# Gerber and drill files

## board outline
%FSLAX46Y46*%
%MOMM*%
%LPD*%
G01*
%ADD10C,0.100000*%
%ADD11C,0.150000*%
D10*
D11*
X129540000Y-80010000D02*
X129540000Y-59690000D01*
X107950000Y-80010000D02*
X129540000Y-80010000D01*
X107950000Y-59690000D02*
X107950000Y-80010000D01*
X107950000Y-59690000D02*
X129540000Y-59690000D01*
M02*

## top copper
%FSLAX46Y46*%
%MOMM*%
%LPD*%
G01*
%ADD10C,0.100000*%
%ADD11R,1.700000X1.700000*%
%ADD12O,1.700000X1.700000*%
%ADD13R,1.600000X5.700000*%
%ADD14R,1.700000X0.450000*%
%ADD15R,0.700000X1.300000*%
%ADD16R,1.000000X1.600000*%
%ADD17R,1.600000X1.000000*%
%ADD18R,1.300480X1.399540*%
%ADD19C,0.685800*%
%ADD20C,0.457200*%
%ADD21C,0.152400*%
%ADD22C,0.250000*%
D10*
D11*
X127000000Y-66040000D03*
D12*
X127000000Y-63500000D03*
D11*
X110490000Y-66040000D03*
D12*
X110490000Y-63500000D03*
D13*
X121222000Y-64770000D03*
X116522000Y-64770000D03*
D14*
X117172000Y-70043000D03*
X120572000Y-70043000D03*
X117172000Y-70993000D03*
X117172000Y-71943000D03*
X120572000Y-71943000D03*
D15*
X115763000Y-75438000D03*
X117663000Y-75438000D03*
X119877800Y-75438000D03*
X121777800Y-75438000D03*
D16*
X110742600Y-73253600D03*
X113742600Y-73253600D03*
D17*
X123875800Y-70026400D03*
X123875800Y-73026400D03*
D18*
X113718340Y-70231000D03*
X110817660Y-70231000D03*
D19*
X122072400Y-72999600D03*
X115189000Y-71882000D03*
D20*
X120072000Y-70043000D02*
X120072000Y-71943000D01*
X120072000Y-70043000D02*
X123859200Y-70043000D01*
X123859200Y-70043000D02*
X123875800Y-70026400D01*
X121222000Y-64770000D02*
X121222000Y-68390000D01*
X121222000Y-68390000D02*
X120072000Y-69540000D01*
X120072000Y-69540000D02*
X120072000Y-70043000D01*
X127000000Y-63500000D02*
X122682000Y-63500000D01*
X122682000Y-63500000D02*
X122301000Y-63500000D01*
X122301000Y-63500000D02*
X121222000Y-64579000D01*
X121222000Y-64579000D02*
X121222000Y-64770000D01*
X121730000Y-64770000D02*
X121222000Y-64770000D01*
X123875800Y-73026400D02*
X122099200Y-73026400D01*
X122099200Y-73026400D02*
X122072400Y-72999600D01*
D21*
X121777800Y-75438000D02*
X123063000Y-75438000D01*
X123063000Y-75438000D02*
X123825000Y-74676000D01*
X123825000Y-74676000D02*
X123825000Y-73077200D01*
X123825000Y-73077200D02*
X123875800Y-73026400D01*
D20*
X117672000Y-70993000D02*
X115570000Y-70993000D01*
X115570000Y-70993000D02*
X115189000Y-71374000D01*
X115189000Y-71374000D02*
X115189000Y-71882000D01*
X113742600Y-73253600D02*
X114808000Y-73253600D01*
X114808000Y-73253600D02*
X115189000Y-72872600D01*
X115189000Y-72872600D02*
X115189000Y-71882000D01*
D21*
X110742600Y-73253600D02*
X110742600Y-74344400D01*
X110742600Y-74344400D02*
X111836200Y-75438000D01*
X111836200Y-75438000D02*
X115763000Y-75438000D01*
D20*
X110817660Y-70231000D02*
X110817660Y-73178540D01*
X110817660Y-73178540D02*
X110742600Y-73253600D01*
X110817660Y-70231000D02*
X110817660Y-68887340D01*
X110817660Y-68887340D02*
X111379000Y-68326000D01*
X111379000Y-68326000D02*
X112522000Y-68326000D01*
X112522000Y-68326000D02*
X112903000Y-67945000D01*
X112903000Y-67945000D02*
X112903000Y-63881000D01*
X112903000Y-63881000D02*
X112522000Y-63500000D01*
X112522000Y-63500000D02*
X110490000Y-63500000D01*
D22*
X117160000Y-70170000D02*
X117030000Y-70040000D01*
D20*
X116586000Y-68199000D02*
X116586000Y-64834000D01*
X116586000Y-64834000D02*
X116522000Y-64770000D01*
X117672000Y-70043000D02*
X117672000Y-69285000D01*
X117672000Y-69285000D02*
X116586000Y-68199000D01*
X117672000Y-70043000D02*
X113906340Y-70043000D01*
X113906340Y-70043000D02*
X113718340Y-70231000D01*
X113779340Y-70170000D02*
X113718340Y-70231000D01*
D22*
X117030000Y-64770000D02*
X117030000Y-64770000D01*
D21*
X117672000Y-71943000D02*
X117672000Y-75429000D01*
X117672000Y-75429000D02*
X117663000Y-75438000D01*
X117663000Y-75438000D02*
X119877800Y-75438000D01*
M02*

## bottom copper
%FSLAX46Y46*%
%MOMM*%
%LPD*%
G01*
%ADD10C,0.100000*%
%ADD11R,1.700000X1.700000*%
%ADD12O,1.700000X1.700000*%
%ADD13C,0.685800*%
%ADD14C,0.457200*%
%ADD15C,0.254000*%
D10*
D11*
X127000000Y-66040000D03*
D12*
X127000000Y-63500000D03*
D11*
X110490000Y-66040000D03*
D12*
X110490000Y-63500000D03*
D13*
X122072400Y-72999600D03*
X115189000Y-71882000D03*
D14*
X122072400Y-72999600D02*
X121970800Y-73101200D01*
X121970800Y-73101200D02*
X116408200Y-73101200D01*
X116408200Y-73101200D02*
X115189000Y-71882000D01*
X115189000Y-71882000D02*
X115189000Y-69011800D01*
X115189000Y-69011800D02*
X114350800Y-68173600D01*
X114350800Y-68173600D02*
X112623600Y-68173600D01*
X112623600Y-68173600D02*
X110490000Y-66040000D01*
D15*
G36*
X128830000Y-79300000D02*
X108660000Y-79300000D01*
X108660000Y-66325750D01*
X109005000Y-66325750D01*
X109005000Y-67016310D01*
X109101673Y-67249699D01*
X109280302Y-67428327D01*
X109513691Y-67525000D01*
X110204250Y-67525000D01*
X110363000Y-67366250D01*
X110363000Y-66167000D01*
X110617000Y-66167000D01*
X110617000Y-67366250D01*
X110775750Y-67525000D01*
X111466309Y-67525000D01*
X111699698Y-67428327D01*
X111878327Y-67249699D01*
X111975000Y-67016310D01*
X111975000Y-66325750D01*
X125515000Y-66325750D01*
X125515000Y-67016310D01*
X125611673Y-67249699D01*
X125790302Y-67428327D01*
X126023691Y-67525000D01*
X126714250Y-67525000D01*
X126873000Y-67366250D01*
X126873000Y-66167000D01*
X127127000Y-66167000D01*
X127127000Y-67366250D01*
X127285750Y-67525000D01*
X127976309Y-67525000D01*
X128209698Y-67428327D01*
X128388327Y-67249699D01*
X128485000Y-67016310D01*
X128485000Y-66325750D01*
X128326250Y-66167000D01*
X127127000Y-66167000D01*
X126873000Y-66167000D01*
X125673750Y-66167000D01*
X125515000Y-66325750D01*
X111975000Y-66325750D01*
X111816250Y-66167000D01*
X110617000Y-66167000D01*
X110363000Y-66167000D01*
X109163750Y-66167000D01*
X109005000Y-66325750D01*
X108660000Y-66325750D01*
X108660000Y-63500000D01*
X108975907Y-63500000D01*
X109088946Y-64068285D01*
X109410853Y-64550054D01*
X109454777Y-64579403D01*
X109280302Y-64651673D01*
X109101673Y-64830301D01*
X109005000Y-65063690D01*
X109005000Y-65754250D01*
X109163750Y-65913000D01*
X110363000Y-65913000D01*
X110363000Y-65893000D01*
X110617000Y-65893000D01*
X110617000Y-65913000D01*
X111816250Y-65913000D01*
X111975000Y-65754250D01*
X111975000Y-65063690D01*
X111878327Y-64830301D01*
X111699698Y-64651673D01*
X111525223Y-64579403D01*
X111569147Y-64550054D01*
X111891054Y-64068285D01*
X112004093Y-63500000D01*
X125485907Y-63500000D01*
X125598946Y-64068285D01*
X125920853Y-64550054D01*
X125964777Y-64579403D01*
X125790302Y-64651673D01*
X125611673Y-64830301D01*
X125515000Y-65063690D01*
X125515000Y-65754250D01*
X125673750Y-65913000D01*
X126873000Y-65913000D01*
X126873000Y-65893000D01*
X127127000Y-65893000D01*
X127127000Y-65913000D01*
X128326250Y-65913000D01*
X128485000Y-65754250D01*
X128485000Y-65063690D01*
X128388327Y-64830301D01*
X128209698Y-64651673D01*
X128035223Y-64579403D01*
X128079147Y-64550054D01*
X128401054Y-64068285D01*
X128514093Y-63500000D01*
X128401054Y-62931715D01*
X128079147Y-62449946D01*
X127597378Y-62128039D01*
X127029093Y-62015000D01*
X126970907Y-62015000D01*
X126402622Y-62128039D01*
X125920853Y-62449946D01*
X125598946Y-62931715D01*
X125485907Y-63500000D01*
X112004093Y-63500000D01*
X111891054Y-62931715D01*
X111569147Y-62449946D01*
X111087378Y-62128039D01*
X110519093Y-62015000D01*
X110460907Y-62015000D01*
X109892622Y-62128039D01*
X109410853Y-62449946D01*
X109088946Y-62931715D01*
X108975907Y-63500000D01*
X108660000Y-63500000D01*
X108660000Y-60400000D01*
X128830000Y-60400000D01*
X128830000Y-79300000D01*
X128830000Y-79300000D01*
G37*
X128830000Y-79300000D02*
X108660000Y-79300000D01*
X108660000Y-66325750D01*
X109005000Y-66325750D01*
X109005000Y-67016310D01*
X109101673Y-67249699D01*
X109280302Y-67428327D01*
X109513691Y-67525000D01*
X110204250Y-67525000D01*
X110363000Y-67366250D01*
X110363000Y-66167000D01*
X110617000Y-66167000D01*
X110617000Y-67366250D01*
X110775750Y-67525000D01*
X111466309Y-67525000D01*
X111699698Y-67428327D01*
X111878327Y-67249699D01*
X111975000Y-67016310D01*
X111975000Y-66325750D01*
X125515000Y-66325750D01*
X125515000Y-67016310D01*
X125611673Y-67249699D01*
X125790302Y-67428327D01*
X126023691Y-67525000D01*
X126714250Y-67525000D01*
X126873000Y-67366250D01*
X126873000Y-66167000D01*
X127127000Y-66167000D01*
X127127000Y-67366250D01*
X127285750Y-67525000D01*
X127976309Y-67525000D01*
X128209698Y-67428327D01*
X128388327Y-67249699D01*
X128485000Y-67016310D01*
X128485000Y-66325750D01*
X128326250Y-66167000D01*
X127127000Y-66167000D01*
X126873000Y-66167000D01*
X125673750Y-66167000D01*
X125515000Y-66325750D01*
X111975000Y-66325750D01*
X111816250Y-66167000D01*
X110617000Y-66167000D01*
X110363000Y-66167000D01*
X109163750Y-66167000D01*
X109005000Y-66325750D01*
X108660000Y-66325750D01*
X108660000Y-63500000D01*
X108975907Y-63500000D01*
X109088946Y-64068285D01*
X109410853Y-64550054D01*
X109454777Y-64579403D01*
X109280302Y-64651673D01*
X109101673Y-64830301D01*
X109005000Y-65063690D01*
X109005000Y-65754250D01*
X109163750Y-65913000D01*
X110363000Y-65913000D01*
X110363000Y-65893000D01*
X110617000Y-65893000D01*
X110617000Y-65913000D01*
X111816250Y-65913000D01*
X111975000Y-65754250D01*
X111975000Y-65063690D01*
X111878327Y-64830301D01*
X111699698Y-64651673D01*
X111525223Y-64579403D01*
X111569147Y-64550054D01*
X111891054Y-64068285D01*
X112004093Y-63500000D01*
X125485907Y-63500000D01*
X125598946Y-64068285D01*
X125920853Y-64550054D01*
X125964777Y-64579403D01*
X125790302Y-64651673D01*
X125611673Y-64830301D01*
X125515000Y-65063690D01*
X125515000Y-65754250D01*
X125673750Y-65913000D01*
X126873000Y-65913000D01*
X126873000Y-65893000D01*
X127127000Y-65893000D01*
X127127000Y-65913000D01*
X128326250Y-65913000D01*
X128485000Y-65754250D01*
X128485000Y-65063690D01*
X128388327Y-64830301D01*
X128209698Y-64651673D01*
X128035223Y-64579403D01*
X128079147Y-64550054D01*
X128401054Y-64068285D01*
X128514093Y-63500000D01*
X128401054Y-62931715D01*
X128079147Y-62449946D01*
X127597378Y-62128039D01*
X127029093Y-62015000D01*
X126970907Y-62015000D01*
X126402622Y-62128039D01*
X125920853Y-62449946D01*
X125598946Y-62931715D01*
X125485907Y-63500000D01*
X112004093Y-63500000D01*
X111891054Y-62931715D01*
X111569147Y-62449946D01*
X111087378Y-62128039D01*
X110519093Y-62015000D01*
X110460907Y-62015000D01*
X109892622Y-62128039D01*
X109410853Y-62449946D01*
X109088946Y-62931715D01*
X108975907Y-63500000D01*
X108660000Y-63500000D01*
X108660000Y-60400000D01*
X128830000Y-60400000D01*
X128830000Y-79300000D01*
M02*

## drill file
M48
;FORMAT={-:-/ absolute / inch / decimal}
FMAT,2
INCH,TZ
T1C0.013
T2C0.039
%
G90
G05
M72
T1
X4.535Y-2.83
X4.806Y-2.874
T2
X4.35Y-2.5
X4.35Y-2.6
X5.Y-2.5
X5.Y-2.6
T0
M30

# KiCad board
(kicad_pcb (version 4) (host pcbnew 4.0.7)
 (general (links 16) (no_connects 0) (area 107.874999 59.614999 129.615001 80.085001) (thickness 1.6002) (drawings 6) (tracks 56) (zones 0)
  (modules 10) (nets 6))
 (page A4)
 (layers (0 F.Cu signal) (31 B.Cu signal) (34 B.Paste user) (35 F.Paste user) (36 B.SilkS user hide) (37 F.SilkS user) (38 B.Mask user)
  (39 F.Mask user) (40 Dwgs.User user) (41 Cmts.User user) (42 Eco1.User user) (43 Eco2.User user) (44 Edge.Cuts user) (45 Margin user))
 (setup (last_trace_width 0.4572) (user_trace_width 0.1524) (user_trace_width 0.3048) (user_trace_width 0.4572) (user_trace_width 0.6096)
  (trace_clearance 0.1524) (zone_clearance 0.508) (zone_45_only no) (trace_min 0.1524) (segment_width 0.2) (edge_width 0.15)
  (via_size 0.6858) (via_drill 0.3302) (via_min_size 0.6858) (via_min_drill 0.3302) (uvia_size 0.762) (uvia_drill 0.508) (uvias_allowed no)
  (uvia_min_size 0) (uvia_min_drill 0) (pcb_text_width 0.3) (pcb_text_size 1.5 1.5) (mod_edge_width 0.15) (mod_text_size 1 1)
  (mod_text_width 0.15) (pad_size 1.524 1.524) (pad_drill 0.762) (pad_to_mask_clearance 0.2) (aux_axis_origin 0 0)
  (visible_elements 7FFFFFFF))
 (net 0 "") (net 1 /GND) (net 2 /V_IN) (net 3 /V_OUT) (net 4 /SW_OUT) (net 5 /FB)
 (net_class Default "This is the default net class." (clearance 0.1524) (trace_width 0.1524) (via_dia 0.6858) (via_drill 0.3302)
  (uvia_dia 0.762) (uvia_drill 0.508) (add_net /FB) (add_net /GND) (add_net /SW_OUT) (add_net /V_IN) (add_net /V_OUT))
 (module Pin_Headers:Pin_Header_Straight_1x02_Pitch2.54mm (layer F.Cu) (at 127 66.04 180)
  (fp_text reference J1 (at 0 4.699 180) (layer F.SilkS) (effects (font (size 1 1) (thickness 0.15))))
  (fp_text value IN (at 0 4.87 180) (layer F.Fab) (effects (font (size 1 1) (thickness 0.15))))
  (pad 1 thru_hole rect (at 0 0 180) (size 1.7 1.7) (drill 1) (layers *.Cu *.Mask) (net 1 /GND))
  (pad 2 thru_hole oval (at 0 2.54 180) (size 1.7 1.7) (drill 1) (layers *.Cu *.Mask) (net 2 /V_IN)))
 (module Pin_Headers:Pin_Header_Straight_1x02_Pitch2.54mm (layer F.Cu) (at 110.49 66.04 180)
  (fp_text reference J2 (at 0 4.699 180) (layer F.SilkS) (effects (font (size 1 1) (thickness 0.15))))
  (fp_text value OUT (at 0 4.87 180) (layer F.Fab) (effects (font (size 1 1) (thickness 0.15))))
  (pad 1 thru_hole rect (at 0 0 180) (size 1.7 1.7) (drill 1) (layers *.Cu *.Mask) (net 1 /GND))
  (pad 2 thru_hole oval (at 0 2.54 180) (size 1.7 1.7) (drill 1) (layers *.Cu *.Mask) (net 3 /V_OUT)))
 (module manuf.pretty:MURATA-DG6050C (layer F.Cu) (at 118.872 64.77 180)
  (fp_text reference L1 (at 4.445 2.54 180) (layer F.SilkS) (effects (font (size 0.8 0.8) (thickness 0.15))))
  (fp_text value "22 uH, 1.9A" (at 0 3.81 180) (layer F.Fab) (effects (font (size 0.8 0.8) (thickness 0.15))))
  (pad 1 smd rect (at -2.35 0 180) (size 1.6 5.7) (layers F.Cu F.Paste F.Mask) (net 2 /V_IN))
  (pad 2 smd rect (at 2.35 0 180) (size 1.6 5.7) (layers F.Cu F.Paste F.Mask) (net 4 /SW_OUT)))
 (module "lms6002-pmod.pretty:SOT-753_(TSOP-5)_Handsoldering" (layer F.Cu) (at 118.872 70.993)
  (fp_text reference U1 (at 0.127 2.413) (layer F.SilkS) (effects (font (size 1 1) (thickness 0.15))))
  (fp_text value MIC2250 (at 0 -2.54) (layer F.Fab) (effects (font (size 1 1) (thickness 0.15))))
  (pad 1 smd rect (at -1.2 -0.95) (size 1.7 0.45) (drill (offset -0.5 0)) (layers F.Cu F.Paste F.Mask) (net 4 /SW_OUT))
  (pad 5 smd rect (at 1.2 -0.95) (size 1.7 0.45) (drill (offset 0.5 0)) (layers F.Cu F.Paste F.Mask) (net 2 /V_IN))
  (pad 2 smd rect (at -1.2 0) (size 1.7 0.45) (drill (offset -0.5 0)) (layers F.Cu F.Paste F.Mask) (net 1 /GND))
  (pad 3 smd rect (at -1.2 0.95) (size 1.7 0.45) (drill (offset -0.5 0)) (layers F.Cu F.Paste F.Mask) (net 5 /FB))
  (pad 4 smd rect (at 1.2 0.95) (size 1.7 0.45) (drill (offset 0.5 0)) (layers F.Cu F.Paste F.Mask) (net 2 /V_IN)))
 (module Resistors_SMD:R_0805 (layer F.Cu) (at 116.713 75.438)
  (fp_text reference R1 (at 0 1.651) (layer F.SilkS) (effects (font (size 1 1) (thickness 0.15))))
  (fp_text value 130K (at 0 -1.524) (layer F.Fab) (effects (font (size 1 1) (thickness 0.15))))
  (pad 1 smd rect (at -0.95 0) (size 0.7 1.3) (layers F.Cu F.Paste F.Mask) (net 3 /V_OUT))
  (pad 2 smd rect (at 0.95 0) (size 0.7 1.3) (layers F.Cu F.Paste F.Mask) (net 5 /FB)))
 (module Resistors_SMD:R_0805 (layer F.Cu) (at 120.8278 75.438)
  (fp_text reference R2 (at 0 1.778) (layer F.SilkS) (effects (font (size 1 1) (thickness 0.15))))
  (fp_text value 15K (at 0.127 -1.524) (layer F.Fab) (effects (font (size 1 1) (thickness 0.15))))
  (pad 1 smd rect (at -0.95 0) (size 0.7 1.3) (layers F.Cu F.Paste F.Mask) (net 5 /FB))
  (pad 2 smd rect (at 0.95 0) (size 0.7 1.3) (layers F.Cu F.Paste F.Mask) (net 1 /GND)))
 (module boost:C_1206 (layer F.Cu) (at 112.2426 73.2536)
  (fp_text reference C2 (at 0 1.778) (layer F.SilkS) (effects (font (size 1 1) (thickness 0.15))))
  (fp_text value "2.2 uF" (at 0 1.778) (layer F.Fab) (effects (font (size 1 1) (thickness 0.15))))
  (pad 1 smd rect (at -1.5 0) (size 1 1.6) (layers F.Cu F.Paste F.Mask) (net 3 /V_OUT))
  (pad 2 smd rect (at 1.5 0) (size 1 1.6) (layers F.Cu F.Paste F.Mask) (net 1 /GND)))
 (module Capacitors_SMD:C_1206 (layer F.Cu) (at 123.8758 71.5264 270)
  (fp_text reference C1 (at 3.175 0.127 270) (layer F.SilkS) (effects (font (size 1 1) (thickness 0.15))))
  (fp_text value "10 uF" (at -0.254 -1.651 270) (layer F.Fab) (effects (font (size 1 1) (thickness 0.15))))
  (pad 1 smd rect (at -1.5 0 270) (size 1 1.6) (layers F.Cu F.Paste F.Mask) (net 2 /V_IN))
  (pad 2 smd rect (at 1.5 0 270) (size 1 1.6) (layers F.Cu F.Paste F.Mask) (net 1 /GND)))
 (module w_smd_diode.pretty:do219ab (layer F.Cu) (at 112.268 70.231)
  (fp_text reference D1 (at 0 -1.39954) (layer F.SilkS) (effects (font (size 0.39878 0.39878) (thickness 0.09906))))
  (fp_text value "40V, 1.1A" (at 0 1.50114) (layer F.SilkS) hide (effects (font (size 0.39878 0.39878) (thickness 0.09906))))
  (pad 2 smd rect (at 1.45034 0) (size 1.30048 1.39954) (layers F.Cu F.Paste F.Mask) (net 4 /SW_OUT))
  (pad 1 smd rect (at -1.45034 0) (size 1.30048 1.39954) (layers F.Cu F.Paste F.Mask) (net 3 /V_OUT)))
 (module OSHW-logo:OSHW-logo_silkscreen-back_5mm (layer B.Cu) (at 125.73 69.85 180)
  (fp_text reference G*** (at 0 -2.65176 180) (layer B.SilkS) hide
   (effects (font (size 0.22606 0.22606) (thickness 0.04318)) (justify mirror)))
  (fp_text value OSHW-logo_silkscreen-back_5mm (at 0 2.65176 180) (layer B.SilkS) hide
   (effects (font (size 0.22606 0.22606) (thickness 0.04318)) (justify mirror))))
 (gr_line (start 129.54 80.01) (end 129.54 59.69) (angle 90) (layer Edge.Cuts) (width 0.15))
 (gr_line (start 107.95 80.01) (end 129.54 80.01) (angle 90) (layer Edge.Cuts) (width 0.15))
 (gr_line (start 107.95 59.69) (end 107.95 80.01) (angle 90) (layer Edge.Cuts) (width 0.15))
 (gr_line (start 107.95 59.69) (end 129.54 59.69) (angle 90) (layer Edge.Cuts) (width 0.15))
 (segment (start 120.072 70.043) (end 120.072 71.943) (width 0.4572) (layer F.Cu) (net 2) (status C00000))
 (segment (start 120.072 70.043) (end 123.8592 70.043) (width 0.4572) (layer F.Cu) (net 2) (status C00000))
 (segment (start 123.8592 70.043) (end 123.8758 70.0264) (width 0.4572) (layer F.Cu) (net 2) (status C00000))
 (segment (start 121.222 64.77) (end 121.222 68.39) (width 0.4572) (layer F.Cu) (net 2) (status 400000))
 (segment (start 121.222 68.39) (end 120.072 69.54) (width 0.4572) (layer F.Cu) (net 2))
 (segment (start 120.072 69.54) (end 120.072 70.043) (width 0.4572) (layer F.Cu) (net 2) (status 800000))
 (segment (start 127 63.5) (end 122.682 63.5) (width 0.4572) (layer F.Cu) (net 2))
 (segment (start 122.682 63.5) (end 122.301 63.5) (width 0.4572) (layer F.Cu) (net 2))
 (segment (start 122.301 63.5) (end 121.222 64.579) (width 0.4572) (layer F.Cu) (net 2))
 (segment (start 121.222 64.579) (end 121.222 64.77) (width 0.4572) (layer F.Cu) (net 2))
 (segment (start 121.73 64.77) (end 121.222 64.77) (width 0.4572) (layer F.Cu) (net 2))
 (segment (start 123.8758 73.0264) (end 122.0992 73.0264) (width 0.4572) (layer F.Cu) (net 1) (status 400000))
 (segment (start 122.0992 73.0264) (end 122.0724 72.9996) (width 0.4572) (layer F.Cu) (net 1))
 (via (at 122.0724 72.9996) (size 0.6858) (drill 0.3302) (layers F.Cu B.Cu) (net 1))
 (segment (start 122.0724 72.9996) (end 121.9708 73.1012) (width 0.4572) (layer B.Cu) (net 1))
 (segment (start 121.9708 73.1012) (end 116.4082 73.1012) (width 0.4572) (layer B.Cu) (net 1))
 (segment (start 116.4082 73.1012) (end 115.189 71.882) (width 0.4572) (layer B.Cu) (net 1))
 (segment (start 121.7778 75.438) (end 123.063 75.438) (width 0.1524) (layer F.Cu) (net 1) (status 400000))
 (segment (start 123.063 75.438) (end 123.825 74.676) (width 0.1524) (layer F.Cu) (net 1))
 (segment (start 123.825 74.676) (end 123.825 73.0772) (width 0.1524) (layer F.Cu) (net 1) (status 800000))
 (segment (start 123.825 73.0772) (end 123.8758 73.0264) (width 0.1524) (layer F.Cu) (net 1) (status C00000))
 (segment (start 117.672 70.993) (end 115.57 70.993) (width 0.4572) (layer F.Cu) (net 1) (status 400000))
 (segment (start 115.57 70.993) (end 115.189 71.374) (width 0.4572) (layer F.Cu) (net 1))
 (segment (start 115.189 71.374) (end 115.189 71.882) (width 0.4572) (layer F.Cu) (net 1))
 (segment (start 113.7426 73.2536) (end 114.808 73.2536) (width 0.4572) (layer F.Cu) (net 1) (status 400000))
 (segment (start 114.808 73.2536) (end 115.189 72.8726) (width 0.4572) (layer F.Cu) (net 1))
 (segment (start 115.189 72.8726) (end 115.189 71.882) (width 0.4572) (layer F.Cu) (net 1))
 (via (at 115.189 71.882) (size 0.6858) (drill 0.3302) (layers F.Cu B.Cu) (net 1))
 (segment (start 115.189 71.882) (end 115.189 69.0118) (width 0.4572) (layer B.Cu) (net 1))
 (segment (start 115.189 69.0118) (end 114.3508 68.1736) (width 0.4572) (layer B.Cu) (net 1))
 (segment (start 114.3508 68.1736) (end 112.6236 68.1736) (width 0.4572) (layer B.Cu) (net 1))
 (segment (start 112.6236 68.1736) (end 110.49 66.04) (width 0.4572) (layer B.Cu) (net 1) (status 800000))
 (segment (start 110.7426 73.2536) (end 110.7426 74.3444) (width 0.1524) (layer F.Cu) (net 3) (status 400000))
 (segment (start 110.7426 74.3444) (end 111.8362 75.438) (width 0.1524) (layer F.Cu) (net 3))
 (segment (start 111.8362 75.438) (end 115.763 75.438) (width 0.1524) (layer F.Cu) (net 3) (status 800000))
 (segment (start 110.81766 70.231) (end 110.81766 73.17854) (width 0.4572) (layer F.Cu) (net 3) (status C00000))
 (segment (start 110.81766 73.17854) (end 110.7426 73.2536) (width 0.4572) (layer F.Cu) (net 3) (status C00000))
 (segment (start 110.81766 70.231) (end 110.81766 68.88734) (width 0.4572) (layer F.Cu) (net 3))
 (segment (start 110.81766 68.88734) (end 111.379 68.326) (width 0.4572) (layer F.Cu) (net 3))
 (segment (start 111.379 68.326) (end 112.522 68.326) (width 0.4572) (layer F.Cu) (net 3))
 (segment (start 112.522 68.326) (end 112.903 67.945) (width 0.4572) (layer F.Cu) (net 3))
 (segment (start 112.903 67.945) (end 112.903 63.881) (width 0.4572) (layer F.Cu) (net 3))
 (segment (start 112.903 63.881) (end 112.522 63.5) (width 0.4572) (layer F.Cu) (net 3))
 (segment (start 112.522 63.5) (end 110.49 63.5) (width 0.4572) (layer F.Cu) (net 3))
 (segment (start 117.16 70.17) (end 117.03 70.04) (width 0.25) (layer F.Cu) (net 4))
 (segment (start 116.586 68.199) (end 116.586 64.834) (width 0.4572) (layer F.Cu) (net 4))
 (segment (start 116.586 64.834) (end 116.522 64.77) (width 0.4572) (layer F.Cu) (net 4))
 (segment (start 117.672 70.043) (end 117.672 69.285) (width 0.4572) (layer F.Cu) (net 4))
 (segment (start 117.672 69.285) (end 116.586 68.199) (width 0.4572) (layer F.Cu) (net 4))
 (segment (start 117.672 70.043) (end 113.90634 70.043) (width 0.4572) (layer F.Cu) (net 4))
 (segment (start 113.90634 70.043) (end 113.71834 70.231) (width 0.4572) (layer F.Cu) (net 4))
 (segment (start 113.77934 70.17) (end 113.71834 70.231) (width 0.4572) (layer F.Cu) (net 4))
 (segment (start 117.03 64.77) (end 117.03 64.77) (width 0.25) (layer F.Cu) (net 4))
 (segment (start 117.672 71.943) (end 117.672 75.429) (width 0.1524) (layer F.Cu) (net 5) (status C00000))
 (segment (start 117.672 75.429) (end 117.663 75.438) (width 0.1524) (layer F.Cu) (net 5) (status C00000))
 (segment (start 117.663 75.438) (end 119.8778 75.438) (width 0.1524) (layer F.Cu) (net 5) (status C00000))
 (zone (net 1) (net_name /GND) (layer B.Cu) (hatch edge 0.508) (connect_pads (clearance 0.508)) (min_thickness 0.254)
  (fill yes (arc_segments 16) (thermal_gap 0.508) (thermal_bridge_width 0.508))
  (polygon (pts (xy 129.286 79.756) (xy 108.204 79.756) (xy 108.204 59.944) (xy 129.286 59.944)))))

